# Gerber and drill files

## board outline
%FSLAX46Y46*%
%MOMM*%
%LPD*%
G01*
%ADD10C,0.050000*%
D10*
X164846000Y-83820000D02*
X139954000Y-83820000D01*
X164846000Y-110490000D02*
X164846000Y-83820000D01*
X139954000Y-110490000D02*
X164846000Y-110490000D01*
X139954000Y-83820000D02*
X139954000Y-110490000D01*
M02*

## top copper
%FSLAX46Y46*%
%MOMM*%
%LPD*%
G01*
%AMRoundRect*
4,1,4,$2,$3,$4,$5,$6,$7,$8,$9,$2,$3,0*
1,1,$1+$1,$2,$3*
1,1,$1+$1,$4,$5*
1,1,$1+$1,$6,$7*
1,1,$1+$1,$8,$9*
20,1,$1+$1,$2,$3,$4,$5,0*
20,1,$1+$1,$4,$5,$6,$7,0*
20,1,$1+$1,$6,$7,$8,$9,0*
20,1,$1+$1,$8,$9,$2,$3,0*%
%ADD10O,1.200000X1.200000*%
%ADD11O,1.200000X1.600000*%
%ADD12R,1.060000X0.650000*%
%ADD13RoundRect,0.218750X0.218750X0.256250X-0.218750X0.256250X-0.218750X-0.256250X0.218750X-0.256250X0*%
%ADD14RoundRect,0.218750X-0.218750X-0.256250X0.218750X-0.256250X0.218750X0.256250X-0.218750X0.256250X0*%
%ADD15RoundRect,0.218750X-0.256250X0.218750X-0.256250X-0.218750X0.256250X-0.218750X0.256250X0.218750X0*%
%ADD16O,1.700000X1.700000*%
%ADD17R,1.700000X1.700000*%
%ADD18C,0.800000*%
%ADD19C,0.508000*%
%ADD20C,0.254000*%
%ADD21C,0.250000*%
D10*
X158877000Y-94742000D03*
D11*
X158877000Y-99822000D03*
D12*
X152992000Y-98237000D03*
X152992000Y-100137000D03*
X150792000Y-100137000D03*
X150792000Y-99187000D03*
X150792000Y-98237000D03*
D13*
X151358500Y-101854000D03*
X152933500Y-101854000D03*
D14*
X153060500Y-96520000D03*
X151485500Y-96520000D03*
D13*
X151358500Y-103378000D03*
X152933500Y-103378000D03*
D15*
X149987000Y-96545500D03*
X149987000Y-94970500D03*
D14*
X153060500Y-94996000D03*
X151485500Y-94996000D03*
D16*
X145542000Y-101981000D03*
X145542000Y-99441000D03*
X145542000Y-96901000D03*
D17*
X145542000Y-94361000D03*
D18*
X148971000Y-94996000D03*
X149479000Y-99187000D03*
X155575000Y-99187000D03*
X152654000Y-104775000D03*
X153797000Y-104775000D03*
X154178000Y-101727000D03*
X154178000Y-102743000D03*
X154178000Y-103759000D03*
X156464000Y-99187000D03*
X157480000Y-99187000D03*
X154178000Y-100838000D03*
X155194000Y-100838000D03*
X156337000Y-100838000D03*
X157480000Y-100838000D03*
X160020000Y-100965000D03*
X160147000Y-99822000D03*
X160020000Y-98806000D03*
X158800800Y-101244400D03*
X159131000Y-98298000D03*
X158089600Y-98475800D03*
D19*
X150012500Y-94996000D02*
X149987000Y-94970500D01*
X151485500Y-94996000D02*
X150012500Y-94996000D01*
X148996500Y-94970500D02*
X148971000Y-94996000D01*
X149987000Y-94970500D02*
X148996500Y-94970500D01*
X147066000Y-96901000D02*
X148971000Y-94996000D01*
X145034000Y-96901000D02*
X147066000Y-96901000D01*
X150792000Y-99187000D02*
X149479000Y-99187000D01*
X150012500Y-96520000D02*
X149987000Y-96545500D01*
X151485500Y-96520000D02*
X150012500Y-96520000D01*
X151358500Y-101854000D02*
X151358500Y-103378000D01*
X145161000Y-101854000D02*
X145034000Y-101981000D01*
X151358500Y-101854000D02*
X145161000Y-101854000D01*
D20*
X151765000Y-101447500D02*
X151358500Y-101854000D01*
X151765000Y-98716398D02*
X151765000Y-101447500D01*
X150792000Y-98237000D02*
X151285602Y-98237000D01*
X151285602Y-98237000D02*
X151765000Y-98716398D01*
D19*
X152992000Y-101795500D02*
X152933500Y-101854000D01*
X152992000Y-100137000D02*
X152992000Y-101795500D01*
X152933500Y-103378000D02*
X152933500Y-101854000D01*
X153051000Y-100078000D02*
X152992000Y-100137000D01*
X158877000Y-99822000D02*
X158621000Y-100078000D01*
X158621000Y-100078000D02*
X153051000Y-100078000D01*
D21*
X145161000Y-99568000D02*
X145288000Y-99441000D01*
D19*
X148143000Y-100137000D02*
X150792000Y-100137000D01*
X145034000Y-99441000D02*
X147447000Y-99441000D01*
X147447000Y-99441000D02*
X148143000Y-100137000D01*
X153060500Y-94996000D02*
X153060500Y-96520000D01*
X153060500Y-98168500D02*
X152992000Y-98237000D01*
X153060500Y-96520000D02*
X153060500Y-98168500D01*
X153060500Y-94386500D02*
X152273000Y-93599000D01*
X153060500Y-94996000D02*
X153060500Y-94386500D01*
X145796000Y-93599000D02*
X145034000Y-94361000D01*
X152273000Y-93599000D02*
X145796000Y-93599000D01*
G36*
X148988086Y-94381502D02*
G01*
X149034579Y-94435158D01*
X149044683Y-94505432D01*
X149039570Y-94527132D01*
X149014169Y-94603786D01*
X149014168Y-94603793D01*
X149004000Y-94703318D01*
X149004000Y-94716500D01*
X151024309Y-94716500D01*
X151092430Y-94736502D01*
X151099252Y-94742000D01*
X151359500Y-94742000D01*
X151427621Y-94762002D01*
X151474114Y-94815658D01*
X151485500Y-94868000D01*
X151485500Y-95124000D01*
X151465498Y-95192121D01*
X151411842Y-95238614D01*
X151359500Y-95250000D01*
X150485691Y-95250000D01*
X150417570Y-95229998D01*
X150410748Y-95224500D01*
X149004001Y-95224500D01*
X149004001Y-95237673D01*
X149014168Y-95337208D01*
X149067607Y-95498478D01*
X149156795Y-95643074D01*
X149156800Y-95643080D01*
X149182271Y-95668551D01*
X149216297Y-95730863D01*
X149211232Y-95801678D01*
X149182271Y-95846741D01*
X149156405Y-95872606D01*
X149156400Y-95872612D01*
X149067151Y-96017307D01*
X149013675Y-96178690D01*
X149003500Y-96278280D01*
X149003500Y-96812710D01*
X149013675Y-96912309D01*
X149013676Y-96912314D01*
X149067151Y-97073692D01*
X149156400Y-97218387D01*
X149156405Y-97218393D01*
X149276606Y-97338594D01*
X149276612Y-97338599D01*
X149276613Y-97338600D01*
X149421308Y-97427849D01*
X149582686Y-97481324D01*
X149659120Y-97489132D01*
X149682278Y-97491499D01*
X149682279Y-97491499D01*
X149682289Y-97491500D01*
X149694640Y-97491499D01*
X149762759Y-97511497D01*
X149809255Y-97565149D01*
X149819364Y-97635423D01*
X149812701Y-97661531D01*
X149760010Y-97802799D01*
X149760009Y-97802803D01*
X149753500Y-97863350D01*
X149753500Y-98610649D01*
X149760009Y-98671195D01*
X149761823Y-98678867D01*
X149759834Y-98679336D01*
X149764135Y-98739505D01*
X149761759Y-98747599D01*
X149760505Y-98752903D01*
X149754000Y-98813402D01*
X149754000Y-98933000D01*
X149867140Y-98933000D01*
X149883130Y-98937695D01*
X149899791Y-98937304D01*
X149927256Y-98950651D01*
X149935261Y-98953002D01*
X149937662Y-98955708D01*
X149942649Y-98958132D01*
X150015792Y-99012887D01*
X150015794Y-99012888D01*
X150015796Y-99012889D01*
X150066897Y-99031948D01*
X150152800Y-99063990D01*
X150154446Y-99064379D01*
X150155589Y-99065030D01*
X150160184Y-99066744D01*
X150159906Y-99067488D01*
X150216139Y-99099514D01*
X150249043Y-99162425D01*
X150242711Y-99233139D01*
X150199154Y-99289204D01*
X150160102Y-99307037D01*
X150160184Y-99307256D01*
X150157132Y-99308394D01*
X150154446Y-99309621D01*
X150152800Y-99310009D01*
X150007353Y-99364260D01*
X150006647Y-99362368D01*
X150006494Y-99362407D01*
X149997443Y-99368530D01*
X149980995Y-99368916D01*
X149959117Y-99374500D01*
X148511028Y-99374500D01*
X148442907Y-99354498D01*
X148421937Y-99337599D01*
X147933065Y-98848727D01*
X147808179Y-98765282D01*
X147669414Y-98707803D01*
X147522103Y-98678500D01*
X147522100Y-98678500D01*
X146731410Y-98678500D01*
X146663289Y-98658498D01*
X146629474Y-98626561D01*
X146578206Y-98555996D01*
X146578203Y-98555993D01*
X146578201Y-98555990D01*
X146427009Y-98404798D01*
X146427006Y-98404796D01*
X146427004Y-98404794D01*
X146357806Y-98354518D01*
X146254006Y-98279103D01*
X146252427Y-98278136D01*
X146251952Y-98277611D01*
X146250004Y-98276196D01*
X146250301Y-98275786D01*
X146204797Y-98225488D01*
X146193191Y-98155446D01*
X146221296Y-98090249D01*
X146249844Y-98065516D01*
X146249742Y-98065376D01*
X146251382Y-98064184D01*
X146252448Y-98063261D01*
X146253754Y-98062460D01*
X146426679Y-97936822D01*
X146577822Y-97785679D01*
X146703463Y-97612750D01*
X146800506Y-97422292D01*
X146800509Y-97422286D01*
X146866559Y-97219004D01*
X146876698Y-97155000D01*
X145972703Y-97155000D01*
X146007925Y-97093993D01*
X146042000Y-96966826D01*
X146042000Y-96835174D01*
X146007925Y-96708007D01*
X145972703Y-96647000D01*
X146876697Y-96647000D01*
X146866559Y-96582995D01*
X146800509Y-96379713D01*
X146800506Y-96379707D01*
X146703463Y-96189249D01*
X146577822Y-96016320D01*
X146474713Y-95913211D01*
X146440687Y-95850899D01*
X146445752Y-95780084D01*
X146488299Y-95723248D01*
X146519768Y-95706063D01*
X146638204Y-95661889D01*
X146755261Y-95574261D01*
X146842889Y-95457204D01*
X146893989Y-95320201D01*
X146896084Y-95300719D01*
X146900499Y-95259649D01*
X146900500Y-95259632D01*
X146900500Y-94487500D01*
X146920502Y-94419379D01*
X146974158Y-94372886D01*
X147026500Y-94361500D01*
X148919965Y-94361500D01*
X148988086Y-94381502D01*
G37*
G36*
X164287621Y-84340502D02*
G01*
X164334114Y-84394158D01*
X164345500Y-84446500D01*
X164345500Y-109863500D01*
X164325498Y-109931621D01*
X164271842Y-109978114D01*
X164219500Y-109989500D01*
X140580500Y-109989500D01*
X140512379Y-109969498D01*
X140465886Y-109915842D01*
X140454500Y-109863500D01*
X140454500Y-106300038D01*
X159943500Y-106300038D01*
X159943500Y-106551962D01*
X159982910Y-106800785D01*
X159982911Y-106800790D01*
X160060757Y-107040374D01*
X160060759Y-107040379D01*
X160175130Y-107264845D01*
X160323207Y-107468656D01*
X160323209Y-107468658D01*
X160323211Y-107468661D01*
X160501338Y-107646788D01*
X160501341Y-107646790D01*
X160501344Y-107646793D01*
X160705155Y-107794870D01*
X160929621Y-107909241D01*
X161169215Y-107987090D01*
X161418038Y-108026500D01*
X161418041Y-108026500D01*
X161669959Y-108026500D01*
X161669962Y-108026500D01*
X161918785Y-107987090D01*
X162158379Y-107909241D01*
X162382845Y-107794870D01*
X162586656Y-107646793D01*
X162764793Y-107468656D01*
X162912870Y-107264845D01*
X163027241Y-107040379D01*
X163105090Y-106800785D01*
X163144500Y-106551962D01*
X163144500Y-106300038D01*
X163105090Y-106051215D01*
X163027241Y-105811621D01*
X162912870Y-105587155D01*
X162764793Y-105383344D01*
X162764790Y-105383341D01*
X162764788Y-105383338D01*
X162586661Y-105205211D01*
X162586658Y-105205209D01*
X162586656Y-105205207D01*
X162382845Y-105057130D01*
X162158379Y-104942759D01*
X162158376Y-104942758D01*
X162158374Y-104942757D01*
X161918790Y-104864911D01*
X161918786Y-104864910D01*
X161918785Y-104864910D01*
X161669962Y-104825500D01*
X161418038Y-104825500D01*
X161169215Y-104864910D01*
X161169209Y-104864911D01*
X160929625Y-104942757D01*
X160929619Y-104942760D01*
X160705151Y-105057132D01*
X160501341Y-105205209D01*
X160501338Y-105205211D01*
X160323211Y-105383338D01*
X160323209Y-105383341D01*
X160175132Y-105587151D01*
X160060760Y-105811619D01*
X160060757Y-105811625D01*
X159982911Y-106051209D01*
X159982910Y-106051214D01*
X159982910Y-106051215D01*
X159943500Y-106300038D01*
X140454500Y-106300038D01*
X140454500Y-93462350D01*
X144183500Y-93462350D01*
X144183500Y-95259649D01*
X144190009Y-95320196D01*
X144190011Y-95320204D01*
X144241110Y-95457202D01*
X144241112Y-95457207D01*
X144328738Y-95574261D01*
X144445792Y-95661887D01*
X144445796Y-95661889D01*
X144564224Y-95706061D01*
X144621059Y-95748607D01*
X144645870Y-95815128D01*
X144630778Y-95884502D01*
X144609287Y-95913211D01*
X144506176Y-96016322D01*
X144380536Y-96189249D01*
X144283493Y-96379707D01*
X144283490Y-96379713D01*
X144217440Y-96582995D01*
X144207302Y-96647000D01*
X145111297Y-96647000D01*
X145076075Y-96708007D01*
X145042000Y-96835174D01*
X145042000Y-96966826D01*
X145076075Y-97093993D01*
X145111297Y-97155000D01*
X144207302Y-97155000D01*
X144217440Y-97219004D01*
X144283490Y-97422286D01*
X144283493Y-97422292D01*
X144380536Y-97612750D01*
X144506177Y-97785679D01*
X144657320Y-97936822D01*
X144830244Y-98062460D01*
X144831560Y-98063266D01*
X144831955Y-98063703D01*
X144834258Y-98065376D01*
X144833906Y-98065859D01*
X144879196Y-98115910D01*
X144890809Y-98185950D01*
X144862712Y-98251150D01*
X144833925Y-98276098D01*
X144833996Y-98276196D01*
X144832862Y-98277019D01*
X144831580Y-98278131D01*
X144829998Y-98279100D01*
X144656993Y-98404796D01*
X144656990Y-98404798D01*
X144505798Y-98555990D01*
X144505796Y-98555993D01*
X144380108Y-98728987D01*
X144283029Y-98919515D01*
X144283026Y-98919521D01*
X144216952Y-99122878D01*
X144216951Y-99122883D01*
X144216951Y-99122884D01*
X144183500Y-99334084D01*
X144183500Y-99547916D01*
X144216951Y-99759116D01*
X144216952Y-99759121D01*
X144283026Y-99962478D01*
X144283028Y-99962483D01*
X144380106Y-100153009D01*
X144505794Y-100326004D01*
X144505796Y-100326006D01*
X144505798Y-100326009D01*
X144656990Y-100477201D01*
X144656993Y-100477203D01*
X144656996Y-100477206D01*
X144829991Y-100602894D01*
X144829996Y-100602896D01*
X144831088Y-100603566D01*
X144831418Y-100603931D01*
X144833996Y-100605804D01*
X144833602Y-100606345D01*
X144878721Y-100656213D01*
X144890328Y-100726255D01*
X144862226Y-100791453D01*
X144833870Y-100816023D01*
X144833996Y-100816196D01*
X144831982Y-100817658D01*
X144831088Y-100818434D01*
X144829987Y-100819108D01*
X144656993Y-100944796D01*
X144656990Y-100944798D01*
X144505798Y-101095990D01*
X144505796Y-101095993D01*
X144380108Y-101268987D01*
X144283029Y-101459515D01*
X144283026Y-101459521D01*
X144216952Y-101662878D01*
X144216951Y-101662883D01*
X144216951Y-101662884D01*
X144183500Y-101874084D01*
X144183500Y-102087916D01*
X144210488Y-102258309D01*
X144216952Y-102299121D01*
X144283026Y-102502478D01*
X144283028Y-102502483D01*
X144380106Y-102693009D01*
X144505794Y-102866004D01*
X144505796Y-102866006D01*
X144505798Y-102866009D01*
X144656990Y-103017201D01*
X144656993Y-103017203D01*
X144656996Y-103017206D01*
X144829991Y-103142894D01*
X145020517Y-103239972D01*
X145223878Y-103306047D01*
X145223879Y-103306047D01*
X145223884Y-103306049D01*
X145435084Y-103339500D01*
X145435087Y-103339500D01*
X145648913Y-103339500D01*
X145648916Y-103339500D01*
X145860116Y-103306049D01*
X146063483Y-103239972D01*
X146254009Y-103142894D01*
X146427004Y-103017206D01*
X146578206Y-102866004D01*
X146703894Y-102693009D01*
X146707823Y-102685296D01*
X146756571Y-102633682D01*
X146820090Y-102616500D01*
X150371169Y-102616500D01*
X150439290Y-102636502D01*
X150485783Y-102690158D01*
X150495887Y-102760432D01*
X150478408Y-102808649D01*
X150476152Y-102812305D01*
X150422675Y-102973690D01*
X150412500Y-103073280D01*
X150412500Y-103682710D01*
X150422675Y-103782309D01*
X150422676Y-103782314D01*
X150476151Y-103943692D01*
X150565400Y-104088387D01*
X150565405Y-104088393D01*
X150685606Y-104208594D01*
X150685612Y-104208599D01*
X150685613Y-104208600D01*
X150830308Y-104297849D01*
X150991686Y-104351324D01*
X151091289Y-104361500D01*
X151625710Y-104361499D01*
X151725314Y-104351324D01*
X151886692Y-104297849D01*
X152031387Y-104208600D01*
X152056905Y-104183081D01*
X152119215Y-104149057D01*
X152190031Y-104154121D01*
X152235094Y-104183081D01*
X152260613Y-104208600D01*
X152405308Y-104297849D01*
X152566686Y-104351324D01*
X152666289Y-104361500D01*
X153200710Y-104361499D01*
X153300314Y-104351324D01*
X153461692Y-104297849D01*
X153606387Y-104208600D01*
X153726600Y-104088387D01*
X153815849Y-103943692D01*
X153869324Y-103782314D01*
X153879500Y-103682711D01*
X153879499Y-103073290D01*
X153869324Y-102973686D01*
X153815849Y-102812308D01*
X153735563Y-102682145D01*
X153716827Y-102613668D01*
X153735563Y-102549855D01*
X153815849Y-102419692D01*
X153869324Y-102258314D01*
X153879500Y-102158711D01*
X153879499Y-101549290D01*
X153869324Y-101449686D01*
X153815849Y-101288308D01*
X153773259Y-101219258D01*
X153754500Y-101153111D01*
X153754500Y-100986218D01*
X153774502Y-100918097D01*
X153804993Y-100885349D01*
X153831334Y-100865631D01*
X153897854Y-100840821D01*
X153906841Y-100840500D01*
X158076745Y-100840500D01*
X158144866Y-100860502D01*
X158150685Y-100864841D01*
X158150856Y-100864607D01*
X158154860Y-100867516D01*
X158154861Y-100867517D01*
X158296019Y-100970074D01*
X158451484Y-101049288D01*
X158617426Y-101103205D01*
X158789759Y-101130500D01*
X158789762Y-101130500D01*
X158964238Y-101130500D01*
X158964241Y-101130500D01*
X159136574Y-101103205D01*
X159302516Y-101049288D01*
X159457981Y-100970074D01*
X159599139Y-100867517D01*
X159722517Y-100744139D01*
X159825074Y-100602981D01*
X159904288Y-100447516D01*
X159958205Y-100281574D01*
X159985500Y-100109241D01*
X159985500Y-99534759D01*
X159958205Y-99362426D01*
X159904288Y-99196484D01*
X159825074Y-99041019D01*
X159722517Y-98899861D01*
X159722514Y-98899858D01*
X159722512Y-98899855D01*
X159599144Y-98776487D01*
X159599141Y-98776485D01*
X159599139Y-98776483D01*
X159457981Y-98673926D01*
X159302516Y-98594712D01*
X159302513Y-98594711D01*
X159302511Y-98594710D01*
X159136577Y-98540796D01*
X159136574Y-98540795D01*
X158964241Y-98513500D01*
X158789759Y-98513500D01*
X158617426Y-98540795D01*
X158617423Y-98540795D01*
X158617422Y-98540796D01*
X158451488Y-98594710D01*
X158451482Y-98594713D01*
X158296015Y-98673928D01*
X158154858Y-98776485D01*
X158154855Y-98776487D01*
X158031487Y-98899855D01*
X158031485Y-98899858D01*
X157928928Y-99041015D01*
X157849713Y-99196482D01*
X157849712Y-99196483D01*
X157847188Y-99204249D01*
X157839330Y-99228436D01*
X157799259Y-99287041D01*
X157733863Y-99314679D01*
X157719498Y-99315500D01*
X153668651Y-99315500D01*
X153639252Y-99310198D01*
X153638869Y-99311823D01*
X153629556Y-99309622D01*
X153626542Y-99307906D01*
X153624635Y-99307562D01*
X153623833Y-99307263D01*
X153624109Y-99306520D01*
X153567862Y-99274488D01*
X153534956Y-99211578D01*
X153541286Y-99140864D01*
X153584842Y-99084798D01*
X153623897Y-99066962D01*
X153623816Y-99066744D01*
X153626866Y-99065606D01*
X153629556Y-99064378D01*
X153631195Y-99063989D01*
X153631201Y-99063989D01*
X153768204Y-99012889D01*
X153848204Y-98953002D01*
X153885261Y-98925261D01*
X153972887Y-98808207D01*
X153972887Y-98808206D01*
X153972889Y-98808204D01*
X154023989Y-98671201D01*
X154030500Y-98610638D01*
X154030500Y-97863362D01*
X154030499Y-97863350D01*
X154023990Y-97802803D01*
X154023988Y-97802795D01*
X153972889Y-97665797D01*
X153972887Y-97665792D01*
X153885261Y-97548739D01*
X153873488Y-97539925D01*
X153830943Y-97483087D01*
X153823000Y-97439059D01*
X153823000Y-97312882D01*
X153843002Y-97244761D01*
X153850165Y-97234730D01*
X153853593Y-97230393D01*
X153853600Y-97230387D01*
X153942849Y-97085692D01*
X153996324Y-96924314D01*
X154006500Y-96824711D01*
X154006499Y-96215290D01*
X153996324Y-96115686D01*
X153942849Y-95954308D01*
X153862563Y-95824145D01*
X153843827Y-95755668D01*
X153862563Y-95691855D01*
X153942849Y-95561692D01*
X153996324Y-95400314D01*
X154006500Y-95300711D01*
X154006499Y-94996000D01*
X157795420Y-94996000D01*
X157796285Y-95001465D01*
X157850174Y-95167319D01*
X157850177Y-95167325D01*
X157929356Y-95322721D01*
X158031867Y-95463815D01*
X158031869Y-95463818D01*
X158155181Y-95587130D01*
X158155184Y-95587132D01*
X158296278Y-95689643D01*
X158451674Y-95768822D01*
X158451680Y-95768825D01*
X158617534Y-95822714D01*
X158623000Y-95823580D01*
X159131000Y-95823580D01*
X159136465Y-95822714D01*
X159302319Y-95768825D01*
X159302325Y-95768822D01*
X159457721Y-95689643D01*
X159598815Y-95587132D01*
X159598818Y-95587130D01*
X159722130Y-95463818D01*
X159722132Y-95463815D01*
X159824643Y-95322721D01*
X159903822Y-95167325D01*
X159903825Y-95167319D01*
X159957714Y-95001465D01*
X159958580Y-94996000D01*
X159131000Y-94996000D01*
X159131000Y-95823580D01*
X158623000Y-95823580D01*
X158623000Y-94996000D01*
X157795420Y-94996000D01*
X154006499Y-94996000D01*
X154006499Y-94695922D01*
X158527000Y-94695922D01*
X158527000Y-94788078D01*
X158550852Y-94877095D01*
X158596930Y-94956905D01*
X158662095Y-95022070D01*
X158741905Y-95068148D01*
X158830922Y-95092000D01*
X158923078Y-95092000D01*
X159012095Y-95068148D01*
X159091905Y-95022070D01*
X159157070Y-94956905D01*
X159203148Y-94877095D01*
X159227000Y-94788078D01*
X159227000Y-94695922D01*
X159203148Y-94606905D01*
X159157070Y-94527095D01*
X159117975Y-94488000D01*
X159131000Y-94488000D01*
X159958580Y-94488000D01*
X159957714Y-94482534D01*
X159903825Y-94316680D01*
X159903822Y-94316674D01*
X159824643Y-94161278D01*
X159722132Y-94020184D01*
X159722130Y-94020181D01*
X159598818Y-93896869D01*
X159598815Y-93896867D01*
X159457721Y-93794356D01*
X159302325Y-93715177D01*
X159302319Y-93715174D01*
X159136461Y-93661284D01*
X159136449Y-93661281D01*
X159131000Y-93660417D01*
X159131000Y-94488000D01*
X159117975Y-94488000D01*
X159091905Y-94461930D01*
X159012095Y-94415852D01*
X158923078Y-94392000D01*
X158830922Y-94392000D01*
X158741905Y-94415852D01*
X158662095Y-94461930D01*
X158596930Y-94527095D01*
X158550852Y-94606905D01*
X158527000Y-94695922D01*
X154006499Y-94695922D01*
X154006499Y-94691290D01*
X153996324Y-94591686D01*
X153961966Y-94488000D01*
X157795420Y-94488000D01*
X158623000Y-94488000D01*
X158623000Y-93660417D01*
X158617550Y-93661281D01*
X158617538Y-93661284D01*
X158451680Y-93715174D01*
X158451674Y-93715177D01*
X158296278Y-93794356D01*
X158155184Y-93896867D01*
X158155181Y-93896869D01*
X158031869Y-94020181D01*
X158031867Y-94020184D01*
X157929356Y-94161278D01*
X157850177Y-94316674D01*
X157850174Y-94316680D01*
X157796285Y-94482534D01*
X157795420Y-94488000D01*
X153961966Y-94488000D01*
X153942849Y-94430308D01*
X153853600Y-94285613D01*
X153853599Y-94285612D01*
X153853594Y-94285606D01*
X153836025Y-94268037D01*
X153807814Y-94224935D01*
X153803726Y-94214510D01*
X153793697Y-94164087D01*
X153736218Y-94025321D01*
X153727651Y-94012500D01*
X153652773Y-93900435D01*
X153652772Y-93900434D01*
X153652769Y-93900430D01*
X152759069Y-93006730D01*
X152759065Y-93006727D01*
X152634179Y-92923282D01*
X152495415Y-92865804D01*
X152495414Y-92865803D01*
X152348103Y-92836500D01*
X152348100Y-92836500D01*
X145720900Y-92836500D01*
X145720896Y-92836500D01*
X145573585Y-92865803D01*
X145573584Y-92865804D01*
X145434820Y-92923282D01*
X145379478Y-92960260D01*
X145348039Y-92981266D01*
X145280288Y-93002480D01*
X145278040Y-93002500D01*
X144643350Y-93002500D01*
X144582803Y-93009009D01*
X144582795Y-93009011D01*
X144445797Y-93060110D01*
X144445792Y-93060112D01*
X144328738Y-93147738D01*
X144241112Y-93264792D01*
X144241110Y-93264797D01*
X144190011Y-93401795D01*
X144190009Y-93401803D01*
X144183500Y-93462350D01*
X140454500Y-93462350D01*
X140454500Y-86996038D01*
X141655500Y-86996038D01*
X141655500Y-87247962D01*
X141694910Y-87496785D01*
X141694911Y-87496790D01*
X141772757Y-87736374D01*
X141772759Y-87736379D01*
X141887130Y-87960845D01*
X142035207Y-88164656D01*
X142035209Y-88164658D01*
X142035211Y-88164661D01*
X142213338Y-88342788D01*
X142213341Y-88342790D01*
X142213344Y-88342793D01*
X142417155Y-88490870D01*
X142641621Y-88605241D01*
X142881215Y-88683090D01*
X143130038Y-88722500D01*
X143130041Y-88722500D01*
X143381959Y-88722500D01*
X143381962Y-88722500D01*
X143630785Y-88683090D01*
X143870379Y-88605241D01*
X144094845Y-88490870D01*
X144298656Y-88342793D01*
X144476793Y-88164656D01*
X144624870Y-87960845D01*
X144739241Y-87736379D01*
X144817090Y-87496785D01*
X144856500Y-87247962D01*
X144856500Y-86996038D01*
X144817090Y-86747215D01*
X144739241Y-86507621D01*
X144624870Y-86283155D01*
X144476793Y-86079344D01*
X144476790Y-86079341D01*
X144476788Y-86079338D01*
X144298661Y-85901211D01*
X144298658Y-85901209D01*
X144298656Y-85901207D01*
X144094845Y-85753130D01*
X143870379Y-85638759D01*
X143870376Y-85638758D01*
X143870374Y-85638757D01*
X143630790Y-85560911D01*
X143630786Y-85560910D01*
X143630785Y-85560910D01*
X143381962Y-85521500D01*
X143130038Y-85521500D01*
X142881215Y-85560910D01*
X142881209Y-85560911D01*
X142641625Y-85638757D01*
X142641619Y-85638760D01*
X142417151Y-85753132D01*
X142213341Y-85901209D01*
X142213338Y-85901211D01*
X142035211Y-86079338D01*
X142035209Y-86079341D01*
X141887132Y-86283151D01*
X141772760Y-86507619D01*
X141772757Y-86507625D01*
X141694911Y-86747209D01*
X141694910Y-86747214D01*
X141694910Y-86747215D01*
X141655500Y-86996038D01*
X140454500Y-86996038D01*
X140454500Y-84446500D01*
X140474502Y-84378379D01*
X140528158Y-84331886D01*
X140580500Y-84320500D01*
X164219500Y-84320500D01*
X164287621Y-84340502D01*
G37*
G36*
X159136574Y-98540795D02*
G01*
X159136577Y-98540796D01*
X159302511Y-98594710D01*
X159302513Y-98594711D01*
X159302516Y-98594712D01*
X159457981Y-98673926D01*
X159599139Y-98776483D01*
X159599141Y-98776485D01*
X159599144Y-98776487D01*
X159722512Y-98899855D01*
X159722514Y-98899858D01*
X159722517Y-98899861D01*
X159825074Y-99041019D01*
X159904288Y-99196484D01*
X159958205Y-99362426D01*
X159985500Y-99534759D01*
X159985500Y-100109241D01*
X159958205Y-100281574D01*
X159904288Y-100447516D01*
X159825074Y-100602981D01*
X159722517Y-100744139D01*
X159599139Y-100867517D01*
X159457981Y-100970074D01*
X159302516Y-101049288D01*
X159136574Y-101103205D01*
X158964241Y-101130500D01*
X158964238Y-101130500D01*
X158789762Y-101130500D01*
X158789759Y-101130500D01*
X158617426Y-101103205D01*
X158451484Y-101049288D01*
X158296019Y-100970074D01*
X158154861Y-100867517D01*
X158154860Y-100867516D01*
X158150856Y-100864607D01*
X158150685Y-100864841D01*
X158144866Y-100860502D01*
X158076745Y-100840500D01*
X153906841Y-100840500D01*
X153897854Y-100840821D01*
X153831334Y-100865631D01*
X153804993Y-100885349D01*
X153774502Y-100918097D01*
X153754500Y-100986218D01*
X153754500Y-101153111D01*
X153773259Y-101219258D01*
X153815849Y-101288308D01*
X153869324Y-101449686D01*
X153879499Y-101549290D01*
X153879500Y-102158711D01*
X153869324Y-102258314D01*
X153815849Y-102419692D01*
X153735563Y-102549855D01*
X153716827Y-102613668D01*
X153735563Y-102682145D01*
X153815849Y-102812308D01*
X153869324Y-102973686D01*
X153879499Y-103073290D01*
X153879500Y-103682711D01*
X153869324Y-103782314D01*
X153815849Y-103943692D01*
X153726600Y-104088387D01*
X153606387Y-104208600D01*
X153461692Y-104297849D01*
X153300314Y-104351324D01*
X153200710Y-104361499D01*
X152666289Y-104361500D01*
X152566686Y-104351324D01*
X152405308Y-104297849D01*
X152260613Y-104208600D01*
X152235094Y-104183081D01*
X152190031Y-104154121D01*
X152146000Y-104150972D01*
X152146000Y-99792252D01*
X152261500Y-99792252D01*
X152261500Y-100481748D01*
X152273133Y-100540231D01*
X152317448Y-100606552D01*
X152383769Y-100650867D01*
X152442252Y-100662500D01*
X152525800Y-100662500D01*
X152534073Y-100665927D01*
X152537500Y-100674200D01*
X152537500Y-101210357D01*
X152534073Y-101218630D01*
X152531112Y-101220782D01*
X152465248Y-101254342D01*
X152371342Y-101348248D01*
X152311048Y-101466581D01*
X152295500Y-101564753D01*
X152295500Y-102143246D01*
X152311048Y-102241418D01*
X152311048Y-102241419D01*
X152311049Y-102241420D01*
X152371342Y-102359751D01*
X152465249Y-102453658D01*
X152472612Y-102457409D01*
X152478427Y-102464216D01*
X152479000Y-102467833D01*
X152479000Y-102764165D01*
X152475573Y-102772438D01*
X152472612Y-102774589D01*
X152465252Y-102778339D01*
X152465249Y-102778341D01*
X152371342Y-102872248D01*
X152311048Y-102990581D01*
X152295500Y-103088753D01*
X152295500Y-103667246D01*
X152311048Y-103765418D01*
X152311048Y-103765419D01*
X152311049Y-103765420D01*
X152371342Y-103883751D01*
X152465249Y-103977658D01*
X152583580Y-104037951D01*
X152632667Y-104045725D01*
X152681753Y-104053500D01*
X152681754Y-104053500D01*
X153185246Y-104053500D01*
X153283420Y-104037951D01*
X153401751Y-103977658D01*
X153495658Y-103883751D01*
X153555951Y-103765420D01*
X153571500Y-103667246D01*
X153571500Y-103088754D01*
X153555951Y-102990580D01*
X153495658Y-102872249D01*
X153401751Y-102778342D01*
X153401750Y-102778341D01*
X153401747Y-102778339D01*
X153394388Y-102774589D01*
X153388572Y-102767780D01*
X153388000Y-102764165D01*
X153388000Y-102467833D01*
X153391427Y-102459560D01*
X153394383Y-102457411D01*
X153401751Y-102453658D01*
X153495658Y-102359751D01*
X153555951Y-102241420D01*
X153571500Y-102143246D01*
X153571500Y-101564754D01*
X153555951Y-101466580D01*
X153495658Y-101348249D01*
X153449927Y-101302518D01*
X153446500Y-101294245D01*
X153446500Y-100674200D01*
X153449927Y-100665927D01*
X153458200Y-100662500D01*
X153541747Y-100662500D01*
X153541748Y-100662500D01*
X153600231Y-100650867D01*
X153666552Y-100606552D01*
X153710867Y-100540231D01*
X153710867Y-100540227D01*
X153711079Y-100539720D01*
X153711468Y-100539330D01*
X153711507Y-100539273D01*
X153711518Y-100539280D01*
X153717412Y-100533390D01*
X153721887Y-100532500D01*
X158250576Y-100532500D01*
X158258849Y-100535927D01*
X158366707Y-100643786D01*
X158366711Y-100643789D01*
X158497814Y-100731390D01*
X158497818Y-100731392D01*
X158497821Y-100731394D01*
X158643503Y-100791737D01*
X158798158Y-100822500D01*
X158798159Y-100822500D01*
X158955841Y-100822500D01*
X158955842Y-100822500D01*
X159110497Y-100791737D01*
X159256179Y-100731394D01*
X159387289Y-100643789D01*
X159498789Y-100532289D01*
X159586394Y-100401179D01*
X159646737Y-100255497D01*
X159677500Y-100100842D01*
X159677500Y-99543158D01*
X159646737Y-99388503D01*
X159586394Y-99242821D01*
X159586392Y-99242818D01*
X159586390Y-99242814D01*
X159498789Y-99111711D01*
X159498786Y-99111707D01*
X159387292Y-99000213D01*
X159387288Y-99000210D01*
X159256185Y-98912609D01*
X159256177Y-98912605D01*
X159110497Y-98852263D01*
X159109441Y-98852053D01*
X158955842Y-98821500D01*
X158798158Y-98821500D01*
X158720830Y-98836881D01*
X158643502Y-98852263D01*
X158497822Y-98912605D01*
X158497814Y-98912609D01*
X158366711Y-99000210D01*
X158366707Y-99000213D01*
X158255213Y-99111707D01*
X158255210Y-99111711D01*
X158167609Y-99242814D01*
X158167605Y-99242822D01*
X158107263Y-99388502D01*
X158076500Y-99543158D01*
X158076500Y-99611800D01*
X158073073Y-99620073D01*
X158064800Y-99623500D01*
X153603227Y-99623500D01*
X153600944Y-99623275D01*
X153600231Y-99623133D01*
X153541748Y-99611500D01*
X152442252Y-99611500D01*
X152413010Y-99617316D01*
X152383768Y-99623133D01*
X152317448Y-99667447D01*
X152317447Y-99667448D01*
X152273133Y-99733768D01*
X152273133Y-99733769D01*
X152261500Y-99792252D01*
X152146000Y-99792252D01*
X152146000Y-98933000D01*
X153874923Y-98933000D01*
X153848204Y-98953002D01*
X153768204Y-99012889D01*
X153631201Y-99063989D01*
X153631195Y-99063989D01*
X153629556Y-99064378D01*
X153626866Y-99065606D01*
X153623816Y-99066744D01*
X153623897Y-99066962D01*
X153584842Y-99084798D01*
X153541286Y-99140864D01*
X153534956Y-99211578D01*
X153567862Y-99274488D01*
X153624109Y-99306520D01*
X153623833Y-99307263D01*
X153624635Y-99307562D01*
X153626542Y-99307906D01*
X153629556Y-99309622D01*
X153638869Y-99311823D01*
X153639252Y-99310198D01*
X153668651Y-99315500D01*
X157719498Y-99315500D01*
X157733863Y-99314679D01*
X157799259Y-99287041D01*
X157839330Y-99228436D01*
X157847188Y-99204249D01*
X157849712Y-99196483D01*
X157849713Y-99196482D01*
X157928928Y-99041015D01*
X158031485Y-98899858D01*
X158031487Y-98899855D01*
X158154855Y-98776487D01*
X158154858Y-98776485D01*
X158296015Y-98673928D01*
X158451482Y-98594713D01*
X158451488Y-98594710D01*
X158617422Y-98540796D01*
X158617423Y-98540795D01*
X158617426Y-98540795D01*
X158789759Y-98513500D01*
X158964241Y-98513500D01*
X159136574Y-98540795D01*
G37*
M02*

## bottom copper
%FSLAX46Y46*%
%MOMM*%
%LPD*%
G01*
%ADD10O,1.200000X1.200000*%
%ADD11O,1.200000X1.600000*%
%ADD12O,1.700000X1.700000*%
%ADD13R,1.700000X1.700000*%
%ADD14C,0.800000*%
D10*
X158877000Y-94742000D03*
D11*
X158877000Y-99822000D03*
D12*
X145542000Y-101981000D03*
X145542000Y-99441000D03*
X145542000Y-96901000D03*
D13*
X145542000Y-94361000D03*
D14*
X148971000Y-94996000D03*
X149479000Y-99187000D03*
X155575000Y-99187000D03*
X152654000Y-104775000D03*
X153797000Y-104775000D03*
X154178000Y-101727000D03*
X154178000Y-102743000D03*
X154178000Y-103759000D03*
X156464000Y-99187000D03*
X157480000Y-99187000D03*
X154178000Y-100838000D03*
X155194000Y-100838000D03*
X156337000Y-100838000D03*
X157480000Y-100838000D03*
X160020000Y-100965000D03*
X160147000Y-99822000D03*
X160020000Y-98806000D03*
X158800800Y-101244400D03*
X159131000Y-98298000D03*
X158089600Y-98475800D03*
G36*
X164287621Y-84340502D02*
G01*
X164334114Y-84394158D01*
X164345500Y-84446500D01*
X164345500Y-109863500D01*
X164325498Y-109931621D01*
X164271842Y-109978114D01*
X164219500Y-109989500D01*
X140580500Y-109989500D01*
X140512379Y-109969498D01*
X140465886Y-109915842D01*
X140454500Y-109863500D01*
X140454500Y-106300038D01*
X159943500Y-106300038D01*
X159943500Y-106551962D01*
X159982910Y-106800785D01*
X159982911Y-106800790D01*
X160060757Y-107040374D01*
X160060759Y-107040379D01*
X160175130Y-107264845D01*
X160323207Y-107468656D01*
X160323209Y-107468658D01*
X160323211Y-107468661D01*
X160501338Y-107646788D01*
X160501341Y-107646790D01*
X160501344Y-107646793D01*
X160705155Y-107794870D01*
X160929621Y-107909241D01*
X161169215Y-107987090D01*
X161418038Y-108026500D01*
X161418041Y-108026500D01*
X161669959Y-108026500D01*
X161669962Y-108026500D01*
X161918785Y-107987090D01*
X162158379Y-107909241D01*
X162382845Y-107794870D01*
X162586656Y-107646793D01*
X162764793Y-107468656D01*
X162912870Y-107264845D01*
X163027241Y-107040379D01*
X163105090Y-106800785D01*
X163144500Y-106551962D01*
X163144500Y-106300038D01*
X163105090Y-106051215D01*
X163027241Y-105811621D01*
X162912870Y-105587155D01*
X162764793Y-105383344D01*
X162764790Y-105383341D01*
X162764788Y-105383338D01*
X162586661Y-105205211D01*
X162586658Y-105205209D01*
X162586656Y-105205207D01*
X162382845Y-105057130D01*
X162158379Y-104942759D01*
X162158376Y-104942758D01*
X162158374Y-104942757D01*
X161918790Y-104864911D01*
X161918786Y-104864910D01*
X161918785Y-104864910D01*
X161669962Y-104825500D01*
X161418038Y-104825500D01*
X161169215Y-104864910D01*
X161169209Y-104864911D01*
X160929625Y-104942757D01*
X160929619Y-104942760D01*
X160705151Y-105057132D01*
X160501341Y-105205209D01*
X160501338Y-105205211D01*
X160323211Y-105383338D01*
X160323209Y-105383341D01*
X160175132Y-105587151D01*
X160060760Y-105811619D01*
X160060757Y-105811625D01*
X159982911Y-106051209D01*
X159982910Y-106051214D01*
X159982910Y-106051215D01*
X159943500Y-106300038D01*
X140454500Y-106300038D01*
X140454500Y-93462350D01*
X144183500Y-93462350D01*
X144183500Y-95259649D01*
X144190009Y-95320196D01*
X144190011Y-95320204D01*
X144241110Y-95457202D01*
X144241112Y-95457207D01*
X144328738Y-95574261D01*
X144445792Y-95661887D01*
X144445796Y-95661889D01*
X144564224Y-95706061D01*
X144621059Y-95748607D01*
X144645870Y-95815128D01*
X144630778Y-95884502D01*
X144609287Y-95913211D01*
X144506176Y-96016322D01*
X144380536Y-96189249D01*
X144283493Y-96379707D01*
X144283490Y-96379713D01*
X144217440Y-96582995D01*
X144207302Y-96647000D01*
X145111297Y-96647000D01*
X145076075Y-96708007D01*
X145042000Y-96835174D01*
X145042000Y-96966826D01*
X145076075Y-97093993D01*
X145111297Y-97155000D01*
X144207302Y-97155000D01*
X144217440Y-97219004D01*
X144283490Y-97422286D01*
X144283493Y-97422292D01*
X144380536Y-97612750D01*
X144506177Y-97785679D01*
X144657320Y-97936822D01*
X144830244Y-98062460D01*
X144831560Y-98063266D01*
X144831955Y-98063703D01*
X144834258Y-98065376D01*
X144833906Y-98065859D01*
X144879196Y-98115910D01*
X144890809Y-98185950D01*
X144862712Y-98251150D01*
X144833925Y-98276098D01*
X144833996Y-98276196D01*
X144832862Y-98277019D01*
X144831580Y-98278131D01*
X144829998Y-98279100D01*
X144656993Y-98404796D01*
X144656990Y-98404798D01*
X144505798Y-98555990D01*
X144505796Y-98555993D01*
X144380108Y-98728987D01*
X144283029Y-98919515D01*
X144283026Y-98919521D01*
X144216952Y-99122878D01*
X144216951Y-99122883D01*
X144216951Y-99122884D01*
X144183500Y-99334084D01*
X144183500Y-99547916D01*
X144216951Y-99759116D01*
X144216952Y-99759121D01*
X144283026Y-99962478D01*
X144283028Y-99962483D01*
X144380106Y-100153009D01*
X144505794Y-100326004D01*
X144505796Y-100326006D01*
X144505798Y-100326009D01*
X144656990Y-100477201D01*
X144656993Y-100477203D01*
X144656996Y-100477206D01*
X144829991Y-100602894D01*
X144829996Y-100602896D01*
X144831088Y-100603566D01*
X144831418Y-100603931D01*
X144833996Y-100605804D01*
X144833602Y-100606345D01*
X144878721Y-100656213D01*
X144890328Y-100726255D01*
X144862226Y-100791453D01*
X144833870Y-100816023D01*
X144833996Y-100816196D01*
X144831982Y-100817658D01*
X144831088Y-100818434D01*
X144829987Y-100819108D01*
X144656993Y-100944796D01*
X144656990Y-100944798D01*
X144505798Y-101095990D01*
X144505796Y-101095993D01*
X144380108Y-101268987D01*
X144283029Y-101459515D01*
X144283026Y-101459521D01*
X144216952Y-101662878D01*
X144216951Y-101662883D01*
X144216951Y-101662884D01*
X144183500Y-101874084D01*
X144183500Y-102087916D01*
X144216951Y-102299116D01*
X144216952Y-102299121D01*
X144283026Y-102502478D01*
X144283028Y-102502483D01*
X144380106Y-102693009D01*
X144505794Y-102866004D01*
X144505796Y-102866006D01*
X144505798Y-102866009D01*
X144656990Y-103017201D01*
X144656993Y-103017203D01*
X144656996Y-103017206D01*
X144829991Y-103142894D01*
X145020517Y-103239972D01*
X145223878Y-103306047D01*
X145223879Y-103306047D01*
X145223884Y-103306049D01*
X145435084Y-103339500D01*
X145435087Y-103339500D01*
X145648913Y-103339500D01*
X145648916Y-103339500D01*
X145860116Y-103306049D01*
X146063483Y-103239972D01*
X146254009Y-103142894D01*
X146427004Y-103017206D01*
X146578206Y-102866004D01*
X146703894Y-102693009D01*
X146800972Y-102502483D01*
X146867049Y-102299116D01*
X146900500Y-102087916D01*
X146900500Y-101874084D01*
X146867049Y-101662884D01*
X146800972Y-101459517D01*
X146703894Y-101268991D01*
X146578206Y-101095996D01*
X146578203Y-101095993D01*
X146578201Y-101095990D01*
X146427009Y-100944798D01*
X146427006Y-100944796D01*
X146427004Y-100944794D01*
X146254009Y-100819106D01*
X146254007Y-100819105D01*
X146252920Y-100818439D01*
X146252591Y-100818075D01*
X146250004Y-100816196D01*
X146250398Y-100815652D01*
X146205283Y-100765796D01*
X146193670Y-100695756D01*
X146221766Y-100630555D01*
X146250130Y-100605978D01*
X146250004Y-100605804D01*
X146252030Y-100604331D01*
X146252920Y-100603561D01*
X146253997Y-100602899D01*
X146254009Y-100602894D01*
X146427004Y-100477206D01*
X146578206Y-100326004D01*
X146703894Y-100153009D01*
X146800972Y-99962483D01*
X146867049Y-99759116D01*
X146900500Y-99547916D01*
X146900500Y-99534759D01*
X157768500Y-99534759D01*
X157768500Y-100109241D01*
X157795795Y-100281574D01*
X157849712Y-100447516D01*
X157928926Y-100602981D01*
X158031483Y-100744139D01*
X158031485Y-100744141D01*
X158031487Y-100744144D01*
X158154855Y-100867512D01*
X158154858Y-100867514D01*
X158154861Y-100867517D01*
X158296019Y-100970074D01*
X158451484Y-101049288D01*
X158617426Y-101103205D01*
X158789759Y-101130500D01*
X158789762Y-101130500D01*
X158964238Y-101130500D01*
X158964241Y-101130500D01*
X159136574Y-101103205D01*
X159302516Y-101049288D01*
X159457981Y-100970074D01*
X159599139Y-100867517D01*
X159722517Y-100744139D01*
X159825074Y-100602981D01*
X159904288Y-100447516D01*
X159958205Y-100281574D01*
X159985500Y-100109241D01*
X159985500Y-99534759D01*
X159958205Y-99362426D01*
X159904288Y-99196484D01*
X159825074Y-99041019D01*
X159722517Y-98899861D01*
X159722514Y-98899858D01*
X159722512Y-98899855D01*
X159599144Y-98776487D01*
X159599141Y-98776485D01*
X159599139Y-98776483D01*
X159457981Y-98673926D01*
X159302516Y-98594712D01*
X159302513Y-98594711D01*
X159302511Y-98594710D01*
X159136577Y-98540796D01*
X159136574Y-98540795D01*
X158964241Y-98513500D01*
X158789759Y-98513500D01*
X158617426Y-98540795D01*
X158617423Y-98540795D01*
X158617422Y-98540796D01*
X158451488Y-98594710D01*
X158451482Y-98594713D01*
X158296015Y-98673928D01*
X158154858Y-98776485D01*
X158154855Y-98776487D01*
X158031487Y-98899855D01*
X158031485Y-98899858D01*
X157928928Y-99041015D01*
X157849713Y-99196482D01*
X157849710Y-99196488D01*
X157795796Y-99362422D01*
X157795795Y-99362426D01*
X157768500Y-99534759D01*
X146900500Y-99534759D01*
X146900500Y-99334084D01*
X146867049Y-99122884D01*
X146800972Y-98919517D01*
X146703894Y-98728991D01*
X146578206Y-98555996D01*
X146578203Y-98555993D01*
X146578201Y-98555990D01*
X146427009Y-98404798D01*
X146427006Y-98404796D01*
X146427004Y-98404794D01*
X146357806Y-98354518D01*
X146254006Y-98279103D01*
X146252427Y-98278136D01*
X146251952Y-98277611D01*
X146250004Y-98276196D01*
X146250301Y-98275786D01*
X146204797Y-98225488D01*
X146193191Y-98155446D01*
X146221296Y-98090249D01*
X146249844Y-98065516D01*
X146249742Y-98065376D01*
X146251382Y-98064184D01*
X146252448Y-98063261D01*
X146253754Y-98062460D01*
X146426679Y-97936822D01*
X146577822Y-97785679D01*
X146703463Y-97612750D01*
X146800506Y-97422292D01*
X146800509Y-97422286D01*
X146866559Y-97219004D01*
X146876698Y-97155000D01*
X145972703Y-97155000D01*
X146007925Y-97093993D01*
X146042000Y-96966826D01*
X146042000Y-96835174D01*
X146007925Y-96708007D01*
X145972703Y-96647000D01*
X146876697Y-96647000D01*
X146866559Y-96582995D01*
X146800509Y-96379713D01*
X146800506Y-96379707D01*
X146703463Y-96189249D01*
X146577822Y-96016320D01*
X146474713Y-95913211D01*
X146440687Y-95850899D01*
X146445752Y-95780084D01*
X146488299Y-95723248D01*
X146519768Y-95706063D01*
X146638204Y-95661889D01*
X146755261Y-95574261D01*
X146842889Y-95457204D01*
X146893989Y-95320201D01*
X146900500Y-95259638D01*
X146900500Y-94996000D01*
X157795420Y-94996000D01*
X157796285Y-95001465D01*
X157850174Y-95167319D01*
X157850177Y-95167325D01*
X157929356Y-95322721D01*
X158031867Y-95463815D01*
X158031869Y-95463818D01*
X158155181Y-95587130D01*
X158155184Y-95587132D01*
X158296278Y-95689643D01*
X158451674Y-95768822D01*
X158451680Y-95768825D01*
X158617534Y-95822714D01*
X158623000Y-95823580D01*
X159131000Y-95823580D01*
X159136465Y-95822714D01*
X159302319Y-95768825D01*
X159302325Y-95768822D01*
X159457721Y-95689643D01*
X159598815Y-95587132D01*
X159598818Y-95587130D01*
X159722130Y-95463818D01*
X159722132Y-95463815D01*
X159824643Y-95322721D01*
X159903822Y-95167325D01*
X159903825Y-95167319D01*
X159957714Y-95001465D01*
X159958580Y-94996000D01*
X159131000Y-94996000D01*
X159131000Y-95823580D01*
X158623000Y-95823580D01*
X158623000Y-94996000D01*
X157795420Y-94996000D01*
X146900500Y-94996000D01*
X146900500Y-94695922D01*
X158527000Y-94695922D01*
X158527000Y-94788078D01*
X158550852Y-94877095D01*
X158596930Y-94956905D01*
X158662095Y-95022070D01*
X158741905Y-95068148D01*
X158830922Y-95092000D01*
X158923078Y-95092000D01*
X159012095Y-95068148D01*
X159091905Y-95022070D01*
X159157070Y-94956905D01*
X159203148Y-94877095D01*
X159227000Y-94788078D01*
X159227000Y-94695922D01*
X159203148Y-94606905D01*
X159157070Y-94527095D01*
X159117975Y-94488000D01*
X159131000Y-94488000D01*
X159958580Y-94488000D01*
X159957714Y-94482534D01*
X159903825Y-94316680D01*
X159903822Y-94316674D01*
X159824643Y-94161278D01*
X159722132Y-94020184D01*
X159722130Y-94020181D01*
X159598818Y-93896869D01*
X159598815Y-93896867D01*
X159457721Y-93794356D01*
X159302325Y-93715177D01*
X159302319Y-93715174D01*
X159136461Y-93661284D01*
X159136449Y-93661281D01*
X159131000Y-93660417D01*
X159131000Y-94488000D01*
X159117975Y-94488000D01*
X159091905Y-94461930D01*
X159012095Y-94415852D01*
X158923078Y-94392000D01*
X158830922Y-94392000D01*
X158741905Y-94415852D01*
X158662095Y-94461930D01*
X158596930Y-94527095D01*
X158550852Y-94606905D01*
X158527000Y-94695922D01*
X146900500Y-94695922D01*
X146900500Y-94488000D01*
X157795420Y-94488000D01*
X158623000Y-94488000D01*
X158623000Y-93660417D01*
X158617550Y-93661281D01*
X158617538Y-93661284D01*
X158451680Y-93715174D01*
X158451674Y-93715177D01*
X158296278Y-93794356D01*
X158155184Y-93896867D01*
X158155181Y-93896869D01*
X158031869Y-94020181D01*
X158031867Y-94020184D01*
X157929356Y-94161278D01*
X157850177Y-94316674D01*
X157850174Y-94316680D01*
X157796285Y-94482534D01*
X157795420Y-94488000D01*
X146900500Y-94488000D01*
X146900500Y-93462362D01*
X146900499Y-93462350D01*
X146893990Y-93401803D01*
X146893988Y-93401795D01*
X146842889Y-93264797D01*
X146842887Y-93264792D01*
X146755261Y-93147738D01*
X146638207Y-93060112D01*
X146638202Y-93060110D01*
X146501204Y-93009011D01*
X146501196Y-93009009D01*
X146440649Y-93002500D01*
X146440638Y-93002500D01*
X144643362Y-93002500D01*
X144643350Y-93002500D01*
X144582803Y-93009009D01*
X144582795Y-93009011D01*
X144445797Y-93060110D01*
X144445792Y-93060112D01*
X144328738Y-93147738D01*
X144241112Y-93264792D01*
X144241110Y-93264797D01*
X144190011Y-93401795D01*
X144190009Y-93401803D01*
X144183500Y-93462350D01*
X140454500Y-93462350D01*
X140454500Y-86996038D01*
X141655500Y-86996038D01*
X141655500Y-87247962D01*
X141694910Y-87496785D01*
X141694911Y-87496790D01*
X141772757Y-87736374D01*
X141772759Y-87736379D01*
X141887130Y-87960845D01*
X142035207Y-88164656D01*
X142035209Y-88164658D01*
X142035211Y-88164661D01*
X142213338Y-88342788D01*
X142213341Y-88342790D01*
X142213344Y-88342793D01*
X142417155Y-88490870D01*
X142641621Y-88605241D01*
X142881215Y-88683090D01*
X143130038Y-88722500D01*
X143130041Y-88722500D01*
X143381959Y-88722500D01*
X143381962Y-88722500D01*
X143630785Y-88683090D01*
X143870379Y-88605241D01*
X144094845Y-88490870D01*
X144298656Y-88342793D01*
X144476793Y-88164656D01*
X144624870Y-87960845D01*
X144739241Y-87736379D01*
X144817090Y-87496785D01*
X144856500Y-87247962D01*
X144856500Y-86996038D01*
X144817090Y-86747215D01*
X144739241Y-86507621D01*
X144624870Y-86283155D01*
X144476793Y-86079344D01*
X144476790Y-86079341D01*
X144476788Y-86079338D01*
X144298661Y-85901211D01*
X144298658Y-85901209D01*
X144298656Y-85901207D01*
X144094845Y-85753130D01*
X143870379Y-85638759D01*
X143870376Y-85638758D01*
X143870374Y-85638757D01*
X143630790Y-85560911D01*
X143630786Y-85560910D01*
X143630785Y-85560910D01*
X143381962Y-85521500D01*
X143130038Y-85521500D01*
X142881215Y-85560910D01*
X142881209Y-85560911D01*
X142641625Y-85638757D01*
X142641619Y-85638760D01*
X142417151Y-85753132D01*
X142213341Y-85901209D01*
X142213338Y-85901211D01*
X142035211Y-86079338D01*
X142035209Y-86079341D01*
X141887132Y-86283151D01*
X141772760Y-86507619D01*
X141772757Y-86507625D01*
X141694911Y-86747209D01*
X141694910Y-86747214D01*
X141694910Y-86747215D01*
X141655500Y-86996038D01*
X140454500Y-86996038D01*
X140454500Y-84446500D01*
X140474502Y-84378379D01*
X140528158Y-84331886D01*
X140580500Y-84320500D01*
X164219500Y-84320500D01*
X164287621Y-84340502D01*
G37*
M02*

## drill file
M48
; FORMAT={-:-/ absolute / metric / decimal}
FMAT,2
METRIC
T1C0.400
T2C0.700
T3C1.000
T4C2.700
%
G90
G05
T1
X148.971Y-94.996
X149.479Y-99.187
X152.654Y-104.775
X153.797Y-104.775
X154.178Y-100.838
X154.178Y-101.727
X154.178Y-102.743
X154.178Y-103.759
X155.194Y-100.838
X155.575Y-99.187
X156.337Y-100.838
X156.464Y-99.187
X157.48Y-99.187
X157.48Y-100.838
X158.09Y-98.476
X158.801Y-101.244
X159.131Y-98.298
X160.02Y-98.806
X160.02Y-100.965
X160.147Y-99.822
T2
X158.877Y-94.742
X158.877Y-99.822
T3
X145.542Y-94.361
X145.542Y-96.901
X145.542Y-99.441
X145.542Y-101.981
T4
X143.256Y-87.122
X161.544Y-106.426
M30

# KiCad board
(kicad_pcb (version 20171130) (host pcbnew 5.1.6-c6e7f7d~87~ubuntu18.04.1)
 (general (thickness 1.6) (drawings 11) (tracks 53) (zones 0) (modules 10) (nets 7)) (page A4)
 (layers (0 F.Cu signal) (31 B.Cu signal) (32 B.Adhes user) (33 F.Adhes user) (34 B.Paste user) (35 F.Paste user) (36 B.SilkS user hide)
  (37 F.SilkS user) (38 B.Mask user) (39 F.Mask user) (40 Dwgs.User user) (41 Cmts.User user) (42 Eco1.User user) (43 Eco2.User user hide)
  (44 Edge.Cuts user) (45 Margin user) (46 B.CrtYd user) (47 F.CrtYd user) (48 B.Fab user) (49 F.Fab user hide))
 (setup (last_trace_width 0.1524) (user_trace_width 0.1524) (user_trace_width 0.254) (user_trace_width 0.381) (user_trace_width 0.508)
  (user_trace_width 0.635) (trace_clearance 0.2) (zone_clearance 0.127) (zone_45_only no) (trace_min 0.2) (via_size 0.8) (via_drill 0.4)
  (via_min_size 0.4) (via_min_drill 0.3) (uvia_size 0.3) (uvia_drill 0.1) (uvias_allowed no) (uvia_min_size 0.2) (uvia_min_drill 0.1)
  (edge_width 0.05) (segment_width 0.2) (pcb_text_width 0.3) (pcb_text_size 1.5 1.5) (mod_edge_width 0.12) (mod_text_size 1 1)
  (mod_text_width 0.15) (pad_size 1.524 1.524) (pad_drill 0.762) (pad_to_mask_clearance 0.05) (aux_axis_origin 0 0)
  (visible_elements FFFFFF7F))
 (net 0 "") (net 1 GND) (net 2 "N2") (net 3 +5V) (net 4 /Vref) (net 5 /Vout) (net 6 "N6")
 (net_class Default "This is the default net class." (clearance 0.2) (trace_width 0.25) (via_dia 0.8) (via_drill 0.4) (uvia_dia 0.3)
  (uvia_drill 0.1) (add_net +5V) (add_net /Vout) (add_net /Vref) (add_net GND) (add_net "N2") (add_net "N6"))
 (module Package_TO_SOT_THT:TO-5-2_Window (layer F.Cu) (at 158.877 99.822 90)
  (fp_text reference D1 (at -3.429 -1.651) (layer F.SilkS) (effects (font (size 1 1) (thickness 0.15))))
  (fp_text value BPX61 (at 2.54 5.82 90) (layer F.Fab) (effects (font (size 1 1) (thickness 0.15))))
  (pad 2 thru_hole oval (at 5.08 0 90) (size 1.2 1.2) (drill 0.7) (layers *.Cu *.Mask) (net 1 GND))
  (pad 1 thru_hole oval (at 0 0 90) (size 1.6 1.2) (drill 0.7) (layers *.Cu *.Mask) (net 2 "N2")))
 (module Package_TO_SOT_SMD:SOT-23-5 (layer F.Cu) (at 151.892 99.187)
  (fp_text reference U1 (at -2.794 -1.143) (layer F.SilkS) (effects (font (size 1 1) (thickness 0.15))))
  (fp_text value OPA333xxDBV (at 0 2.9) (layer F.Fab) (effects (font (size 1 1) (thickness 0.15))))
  (pad 5 smd rect (at 1.1 -0.95) (size 1.06 0.65) (layers F.Cu F.Paste F.Mask) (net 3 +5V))
  (pad 4 smd rect (at 1.1 0.95) (size 1.06 0.65) (layers F.Cu F.Paste F.Mask) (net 2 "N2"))
  (pad 3 smd rect (at -1.1 0.95) (size 1.06 0.65) (layers F.Cu F.Paste F.Mask) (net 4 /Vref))
  (pad 2 smd rect (at -1.1 0) (size 1.06 0.65) (layers F.Cu F.Paste F.Mask) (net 1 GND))
  (pad 1 smd rect (at -1.1 -0.95) (size 1.06 0.65) (layers F.Cu F.Paste F.Mask) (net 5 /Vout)))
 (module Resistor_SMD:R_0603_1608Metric (layer F.Cu) (at 152.146 101.854 180)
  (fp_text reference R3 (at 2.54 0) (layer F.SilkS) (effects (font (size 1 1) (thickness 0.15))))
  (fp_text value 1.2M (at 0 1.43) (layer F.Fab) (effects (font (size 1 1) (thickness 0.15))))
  (pad 2 smd roundrect (at 0.7875 0 180) (size 0.875 0.95) (layers F.Cu F.Paste F.Mask) (roundrect_rratio 0.25) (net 5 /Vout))
  (pad 1 smd roundrect (at -0.7875 0 180) (size 0.875 0.95) (layers F.Cu F.Paste F.Mask) (roundrect_rratio 0.25) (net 2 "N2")))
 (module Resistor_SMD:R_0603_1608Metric (layer F.Cu) (at 152.273 96.52)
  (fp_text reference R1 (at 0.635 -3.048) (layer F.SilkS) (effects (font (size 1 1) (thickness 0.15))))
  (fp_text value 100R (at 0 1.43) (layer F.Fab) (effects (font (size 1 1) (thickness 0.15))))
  (pad 2 smd roundrect (at 0.7875 0) (size 0.875 0.95) (layers F.Cu F.Paste F.Mask) (roundrect_rratio 0.25) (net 3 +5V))
  (pad 1 smd roundrect (at -0.7875 0) (size 0.875 0.95) (layers F.Cu F.Paste F.Mask) (roundrect_rratio 0.25) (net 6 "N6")))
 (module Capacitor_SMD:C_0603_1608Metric (layer F.Cu) (at 152.146 103.378 180)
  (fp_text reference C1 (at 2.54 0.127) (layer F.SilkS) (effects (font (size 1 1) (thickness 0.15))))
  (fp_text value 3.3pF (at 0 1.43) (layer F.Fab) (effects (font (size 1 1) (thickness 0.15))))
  (pad 2 smd roundrect (at 0.7875 0 180) (size 0.875 0.95) (layers F.Cu F.Paste F.Mask) (roundrect_rratio 0.25) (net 5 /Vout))
  (pad 1 smd roundrect (at -0.7875 0 180) (size 0.875 0.95) (layers F.Cu F.Paste F.Mask) (roundrect_rratio 0.25) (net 2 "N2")))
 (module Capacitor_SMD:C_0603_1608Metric (layer F.Cu) (at 149.987 95.758 270)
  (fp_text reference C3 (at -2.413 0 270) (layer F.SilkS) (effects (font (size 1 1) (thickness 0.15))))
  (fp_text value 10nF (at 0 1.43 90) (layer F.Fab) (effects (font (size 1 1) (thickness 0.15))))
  (pad 2 smd roundrect (at 0.7875 0 270) (size 0.875 0.95) (layers F.Cu F.Paste F.Mask) (roundrect_rratio 0.25) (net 6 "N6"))
  (pad 1 smd roundrect (at -0.7875 0 270) (size 0.875 0.95) (layers F.Cu F.Paste F.Mask) (roundrect_rratio 0.25) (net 1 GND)))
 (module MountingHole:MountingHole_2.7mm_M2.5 (layer F.Cu) (at 161.544 106.426)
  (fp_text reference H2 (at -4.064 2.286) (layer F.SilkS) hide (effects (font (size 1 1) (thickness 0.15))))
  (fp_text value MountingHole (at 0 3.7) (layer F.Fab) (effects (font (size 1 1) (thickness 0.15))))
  (pad 1 np_thru_hole circle (at 0 0) (size 2.7 2.7) (drill 2.7) (layers *.Cu *.Mask)))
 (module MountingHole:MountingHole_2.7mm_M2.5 (layer F.Cu) (at 143.256 87.122)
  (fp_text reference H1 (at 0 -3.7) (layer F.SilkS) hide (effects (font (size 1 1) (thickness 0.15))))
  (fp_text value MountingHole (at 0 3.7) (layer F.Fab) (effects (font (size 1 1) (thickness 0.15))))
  (pad 1 np_thru_hole circle (at 0 0) (size 2.7 2.7) (drill 2.7) (layers *.Cu *.Mask)))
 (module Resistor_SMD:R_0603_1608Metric (layer F.Cu) (at 152.273 94.996)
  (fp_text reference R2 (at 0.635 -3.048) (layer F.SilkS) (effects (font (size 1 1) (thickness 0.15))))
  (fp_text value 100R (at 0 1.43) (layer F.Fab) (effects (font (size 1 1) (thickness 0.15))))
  (pad 2 smd roundrect (at 0.7875 0) (size 0.875 0.95) (layers F.Cu F.Paste F.Mask) (roundrect_rratio 0.25) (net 3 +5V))
  (pad 1 smd roundrect (at -0.7875 0) (size 0.875 0.95) (layers F.Cu F.Paste F.Mask) (roundrect_rratio 0.25) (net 1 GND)))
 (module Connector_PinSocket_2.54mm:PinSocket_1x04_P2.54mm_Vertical (layer F.Cu) (at 145.542 94.361)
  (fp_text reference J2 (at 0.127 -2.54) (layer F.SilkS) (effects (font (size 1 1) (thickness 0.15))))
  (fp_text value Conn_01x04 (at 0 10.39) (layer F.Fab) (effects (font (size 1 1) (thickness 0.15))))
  (pad 4 thru_hole oval (at 0 7.62) (size 1.7 1.7) (drill 1) (layers *.Cu *.Mask) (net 5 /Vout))
  (pad 3 thru_hole oval (at 0 5.08) (size 1.7 1.7) (drill 1) (layers *.Cu *.Mask) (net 4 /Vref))
  (pad 2 thru_hole oval (at 0 2.54) (size 1.7 1.7) (drill 1) (layers *.Cu *.Mask) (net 1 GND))
  (pad 1 thru_hole rect (at 0 0) (size 1.7 1.7) (drill 1) (layers *.Cu *.Mask) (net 3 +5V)))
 (gr_line (start 164.846 83.82) (end 139.954 83.82) (layer Edge.Cuts) (width 0.05))
 (gr_line (start 164.846 110.49) (end 164.846 83.82) (layer Edge.Cuts) (width 0.05))
 (gr_line (start 139.954 110.49) (end 164.846 110.49) (layer Edge.Cuts) (width 0.05))
 (gr_line (start 139.954 83.82) (end 139.954 110.49) (layer Edge.Cuts) (width 0.05))
 (segment (start 150.0125 94.996) (end 149.987 94.9705) (width 0.508) (layer F.Cu) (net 1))
 (segment (start 151.4855 94.996) (end 150.0125 94.996) (width 0.508) (layer F.Cu) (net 1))
 (via (at 148.971 94.996) (size 0.8) (drill 0.4) (layers F.Cu B.Cu) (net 1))
 (segment (start 148.9965 94.9705) (end 148.971 94.996) (width 0.508) (layer F.Cu) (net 1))
 (segment (start 149.987 94.9705) (end 148.9965 94.9705) (width 0.508) (layer F.Cu) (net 1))
 (segment (start 147.066 96.901) (end 148.971 94.996) (width 0.508) (layer F.Cu) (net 1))
 (segment (start 145.034 96.901) (end 147.066 96.901) (width 0.508) (layer F.Cu) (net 1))
 (via (at 149.479 99.187) (size 0.8) (drill 0.4) (layers F.Cu B.Cu) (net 1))
 (segment (start 150.792 99.187) (end 149.479 99.187) (width 0.508) (layer F.Cu) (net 1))
 (via (at 155.575 99.187) (size 0.8) (drill 0.4) (layers F.Cu B.Cu) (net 1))
 (via (at 152.654 104.775) (size 0.8) (drill 0.4) (layers F.Cu B.Cu) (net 1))
 (via (at 153.797 104.775) (size 0.8) (drill 0.4) (layers F.Cu B.Cu) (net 1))
 (via (at 154.178 101.727) (size 0.8) (drill 0.4) (layers F.Cu B.Cu) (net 1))
 (via (at 154.178 102.743) (size 0.8) (drill 0.4) (layers F.Cu B.Cu) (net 1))
 (via (at 154.178 103.759) (size 0.8) (drill 0.4) (layers F.Cu B.Cu) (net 1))
 (via (at 156.464 99.187) (size 0.8) (drill 0.4) (layers F.Cu B.Cu) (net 1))
 (via (at 157.48 99.187) (size 0.8) (drill 0.4) (layers F.Cu B.Cu) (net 1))
 (via (at 154.178 100.838) (size 0.8) (drill 0.4) (layers F.Cu B.Cu) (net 1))
 (via (at 155.194 100.838) (size 0.8) (drill 0.4) (layers F.Cu B.Cu) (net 1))
 (via (at 156.337 100.838) (size 0.8) (drill 0.4) (layers F.Cu B.Cu) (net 1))
 (via (at 157.48 100.838) (size 0.8) (drill 0.4) (layers F.Cu B.Cu) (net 1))
 (via (at 160.02 100.965) (size 0.8) (drill 0.4) (layers F.Cu B.Cu) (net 1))
 (via (at 160.147 99.822) (size 0.8) (drill 0.4) (layers F.Cu B.Cu) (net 1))
 (via (at 160.02 98.806) (size 0.8) (drill 0.4) (layers F.Cu B.Cu) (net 1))
 (via (at 158.8008 101.2444) (size 0.8) (drill 0.4) (layers F.Cu B.Cu) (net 1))
 (via (at 159.131 98.298) (size 0.8) (drill 0.4) (layers F.Cu B.Cu) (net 1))
 (via (at 158.0896 98.4758) (size 0.8) (drill 0.4) (layers F.Cu B.Cu) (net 1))
 (segment (start 150.0125 96.52) (end 149.987 96.5455) (width 0.508) (layer F.Cu) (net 6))
 (segment (start 151.4855 96.52) (end 150.0125 96.52) (width 0.508) (layer F.Cu) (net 6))
 (segment (start 151.3585 101.854) (end 151.3585 103.378) (width 0.508) (layer F.Cu) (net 5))
 (segment (start 145.161 101.854) (end 145.034 101.981) (width 0.508) (layer F.Cu) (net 5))
 (segment (start 151.3585 101.854) (end 145.161 101.854) (width 0.508) (layer F.Cu) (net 5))
 (segment (start 151.765 101.4475) (end 151.3585 101.854) (width 0.254) (layer F.Cu) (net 5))
 (segment (start 151.765 98.716398) (end 151.765 101.4475) (width 0.254) (layer F.Cu) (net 5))
 (segment (start 150.792 98.237) (end 151.285602 98.237) (width 0.254) (layer F.Cu) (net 5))
 (segment (start 151.285602 98.237) (end 151.765 98.716398) (width 0.254) (layer F.Cu) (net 5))
 (segment (start 152.992 101.7955) (end 152.9335 101.854) (width 0.508) (layer F.Cu) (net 2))
 (segment (start 152.992 100.137) (end 152.992 101.7955) (width 0.508) (layer F.Cu) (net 2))
 (segment (start 152.9335 103.378) (end 152.9335 101.854) (width 0.508) (layer F.Cu) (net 2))
 (segment (start 153.051 100.078) (end 152.992 100.137) (width 0.508) (layer F.Cu) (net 2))
 (segment (start 158.877 99.822) (end 158.621 100.078) (width 0.508) (layer F.Cu) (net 2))
 (segment (start 158.621 100.078) (end 153.051 100.078) (width 0.508) (layer F.Cu) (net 2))
 (segment (start 145.161 99.568) (end 145.288 99.441) (width 0.25) (layer F.Cu) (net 4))
 (segment (start 148.143 100.137) (end 150.792 100.137) (width 0.508) (layer F.Cu) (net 4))
 (segment (start 145.034 99.441) (end 147.447 99.441) (width 0.508) (layer F.Cu) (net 4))
 (segment (start 147.447 99.441) (end 148.143 100.137) (width 0.508) (layer F.Cu) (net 4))
 (segment (start 153.0605 94.996) (end 153.0605 96.52) (width 0.508) (layer F.Cu) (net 3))
 (segment (start 153.0605 98.1685) (end 152.992 98.237) (width 0.508) (layer F.Cu) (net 3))
 (segment (start 153.0605 96.52) (end 153.0605 98.1685) (width 0.508) (layer F.Cu) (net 3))
 (segment (start 153.0605 94.3865) (end 152.273 93.599) (width 0.508) (layer F.Cu) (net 3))
 (segment (start 153.0605 94.996) (end 153.0605 94.3865) (width 0.508) (layer F.Cu) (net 3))
 (segment (start 145.796 93.599) (end 145.034 94.361) (width 0.508) (layer F.Cu) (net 3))
 (segment (start 152.273 93.599) (end 145.796 93.599) (width 0.508) (layer F.Cu) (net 3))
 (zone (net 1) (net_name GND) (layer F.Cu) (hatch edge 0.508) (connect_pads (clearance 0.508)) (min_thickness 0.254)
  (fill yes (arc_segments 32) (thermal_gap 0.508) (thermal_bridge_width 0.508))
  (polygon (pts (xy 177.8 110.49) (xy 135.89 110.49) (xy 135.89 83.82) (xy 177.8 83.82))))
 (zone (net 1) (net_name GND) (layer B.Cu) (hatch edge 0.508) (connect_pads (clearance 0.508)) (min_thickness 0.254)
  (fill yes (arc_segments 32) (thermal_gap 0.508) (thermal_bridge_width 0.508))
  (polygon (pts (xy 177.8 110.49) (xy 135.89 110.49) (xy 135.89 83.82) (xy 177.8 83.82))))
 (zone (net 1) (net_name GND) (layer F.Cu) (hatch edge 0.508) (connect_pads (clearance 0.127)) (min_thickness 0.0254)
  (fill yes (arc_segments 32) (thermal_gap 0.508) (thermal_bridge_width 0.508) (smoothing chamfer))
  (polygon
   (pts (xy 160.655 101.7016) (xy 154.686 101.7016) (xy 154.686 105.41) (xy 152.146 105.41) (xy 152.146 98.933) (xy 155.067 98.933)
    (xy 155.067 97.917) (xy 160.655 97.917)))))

